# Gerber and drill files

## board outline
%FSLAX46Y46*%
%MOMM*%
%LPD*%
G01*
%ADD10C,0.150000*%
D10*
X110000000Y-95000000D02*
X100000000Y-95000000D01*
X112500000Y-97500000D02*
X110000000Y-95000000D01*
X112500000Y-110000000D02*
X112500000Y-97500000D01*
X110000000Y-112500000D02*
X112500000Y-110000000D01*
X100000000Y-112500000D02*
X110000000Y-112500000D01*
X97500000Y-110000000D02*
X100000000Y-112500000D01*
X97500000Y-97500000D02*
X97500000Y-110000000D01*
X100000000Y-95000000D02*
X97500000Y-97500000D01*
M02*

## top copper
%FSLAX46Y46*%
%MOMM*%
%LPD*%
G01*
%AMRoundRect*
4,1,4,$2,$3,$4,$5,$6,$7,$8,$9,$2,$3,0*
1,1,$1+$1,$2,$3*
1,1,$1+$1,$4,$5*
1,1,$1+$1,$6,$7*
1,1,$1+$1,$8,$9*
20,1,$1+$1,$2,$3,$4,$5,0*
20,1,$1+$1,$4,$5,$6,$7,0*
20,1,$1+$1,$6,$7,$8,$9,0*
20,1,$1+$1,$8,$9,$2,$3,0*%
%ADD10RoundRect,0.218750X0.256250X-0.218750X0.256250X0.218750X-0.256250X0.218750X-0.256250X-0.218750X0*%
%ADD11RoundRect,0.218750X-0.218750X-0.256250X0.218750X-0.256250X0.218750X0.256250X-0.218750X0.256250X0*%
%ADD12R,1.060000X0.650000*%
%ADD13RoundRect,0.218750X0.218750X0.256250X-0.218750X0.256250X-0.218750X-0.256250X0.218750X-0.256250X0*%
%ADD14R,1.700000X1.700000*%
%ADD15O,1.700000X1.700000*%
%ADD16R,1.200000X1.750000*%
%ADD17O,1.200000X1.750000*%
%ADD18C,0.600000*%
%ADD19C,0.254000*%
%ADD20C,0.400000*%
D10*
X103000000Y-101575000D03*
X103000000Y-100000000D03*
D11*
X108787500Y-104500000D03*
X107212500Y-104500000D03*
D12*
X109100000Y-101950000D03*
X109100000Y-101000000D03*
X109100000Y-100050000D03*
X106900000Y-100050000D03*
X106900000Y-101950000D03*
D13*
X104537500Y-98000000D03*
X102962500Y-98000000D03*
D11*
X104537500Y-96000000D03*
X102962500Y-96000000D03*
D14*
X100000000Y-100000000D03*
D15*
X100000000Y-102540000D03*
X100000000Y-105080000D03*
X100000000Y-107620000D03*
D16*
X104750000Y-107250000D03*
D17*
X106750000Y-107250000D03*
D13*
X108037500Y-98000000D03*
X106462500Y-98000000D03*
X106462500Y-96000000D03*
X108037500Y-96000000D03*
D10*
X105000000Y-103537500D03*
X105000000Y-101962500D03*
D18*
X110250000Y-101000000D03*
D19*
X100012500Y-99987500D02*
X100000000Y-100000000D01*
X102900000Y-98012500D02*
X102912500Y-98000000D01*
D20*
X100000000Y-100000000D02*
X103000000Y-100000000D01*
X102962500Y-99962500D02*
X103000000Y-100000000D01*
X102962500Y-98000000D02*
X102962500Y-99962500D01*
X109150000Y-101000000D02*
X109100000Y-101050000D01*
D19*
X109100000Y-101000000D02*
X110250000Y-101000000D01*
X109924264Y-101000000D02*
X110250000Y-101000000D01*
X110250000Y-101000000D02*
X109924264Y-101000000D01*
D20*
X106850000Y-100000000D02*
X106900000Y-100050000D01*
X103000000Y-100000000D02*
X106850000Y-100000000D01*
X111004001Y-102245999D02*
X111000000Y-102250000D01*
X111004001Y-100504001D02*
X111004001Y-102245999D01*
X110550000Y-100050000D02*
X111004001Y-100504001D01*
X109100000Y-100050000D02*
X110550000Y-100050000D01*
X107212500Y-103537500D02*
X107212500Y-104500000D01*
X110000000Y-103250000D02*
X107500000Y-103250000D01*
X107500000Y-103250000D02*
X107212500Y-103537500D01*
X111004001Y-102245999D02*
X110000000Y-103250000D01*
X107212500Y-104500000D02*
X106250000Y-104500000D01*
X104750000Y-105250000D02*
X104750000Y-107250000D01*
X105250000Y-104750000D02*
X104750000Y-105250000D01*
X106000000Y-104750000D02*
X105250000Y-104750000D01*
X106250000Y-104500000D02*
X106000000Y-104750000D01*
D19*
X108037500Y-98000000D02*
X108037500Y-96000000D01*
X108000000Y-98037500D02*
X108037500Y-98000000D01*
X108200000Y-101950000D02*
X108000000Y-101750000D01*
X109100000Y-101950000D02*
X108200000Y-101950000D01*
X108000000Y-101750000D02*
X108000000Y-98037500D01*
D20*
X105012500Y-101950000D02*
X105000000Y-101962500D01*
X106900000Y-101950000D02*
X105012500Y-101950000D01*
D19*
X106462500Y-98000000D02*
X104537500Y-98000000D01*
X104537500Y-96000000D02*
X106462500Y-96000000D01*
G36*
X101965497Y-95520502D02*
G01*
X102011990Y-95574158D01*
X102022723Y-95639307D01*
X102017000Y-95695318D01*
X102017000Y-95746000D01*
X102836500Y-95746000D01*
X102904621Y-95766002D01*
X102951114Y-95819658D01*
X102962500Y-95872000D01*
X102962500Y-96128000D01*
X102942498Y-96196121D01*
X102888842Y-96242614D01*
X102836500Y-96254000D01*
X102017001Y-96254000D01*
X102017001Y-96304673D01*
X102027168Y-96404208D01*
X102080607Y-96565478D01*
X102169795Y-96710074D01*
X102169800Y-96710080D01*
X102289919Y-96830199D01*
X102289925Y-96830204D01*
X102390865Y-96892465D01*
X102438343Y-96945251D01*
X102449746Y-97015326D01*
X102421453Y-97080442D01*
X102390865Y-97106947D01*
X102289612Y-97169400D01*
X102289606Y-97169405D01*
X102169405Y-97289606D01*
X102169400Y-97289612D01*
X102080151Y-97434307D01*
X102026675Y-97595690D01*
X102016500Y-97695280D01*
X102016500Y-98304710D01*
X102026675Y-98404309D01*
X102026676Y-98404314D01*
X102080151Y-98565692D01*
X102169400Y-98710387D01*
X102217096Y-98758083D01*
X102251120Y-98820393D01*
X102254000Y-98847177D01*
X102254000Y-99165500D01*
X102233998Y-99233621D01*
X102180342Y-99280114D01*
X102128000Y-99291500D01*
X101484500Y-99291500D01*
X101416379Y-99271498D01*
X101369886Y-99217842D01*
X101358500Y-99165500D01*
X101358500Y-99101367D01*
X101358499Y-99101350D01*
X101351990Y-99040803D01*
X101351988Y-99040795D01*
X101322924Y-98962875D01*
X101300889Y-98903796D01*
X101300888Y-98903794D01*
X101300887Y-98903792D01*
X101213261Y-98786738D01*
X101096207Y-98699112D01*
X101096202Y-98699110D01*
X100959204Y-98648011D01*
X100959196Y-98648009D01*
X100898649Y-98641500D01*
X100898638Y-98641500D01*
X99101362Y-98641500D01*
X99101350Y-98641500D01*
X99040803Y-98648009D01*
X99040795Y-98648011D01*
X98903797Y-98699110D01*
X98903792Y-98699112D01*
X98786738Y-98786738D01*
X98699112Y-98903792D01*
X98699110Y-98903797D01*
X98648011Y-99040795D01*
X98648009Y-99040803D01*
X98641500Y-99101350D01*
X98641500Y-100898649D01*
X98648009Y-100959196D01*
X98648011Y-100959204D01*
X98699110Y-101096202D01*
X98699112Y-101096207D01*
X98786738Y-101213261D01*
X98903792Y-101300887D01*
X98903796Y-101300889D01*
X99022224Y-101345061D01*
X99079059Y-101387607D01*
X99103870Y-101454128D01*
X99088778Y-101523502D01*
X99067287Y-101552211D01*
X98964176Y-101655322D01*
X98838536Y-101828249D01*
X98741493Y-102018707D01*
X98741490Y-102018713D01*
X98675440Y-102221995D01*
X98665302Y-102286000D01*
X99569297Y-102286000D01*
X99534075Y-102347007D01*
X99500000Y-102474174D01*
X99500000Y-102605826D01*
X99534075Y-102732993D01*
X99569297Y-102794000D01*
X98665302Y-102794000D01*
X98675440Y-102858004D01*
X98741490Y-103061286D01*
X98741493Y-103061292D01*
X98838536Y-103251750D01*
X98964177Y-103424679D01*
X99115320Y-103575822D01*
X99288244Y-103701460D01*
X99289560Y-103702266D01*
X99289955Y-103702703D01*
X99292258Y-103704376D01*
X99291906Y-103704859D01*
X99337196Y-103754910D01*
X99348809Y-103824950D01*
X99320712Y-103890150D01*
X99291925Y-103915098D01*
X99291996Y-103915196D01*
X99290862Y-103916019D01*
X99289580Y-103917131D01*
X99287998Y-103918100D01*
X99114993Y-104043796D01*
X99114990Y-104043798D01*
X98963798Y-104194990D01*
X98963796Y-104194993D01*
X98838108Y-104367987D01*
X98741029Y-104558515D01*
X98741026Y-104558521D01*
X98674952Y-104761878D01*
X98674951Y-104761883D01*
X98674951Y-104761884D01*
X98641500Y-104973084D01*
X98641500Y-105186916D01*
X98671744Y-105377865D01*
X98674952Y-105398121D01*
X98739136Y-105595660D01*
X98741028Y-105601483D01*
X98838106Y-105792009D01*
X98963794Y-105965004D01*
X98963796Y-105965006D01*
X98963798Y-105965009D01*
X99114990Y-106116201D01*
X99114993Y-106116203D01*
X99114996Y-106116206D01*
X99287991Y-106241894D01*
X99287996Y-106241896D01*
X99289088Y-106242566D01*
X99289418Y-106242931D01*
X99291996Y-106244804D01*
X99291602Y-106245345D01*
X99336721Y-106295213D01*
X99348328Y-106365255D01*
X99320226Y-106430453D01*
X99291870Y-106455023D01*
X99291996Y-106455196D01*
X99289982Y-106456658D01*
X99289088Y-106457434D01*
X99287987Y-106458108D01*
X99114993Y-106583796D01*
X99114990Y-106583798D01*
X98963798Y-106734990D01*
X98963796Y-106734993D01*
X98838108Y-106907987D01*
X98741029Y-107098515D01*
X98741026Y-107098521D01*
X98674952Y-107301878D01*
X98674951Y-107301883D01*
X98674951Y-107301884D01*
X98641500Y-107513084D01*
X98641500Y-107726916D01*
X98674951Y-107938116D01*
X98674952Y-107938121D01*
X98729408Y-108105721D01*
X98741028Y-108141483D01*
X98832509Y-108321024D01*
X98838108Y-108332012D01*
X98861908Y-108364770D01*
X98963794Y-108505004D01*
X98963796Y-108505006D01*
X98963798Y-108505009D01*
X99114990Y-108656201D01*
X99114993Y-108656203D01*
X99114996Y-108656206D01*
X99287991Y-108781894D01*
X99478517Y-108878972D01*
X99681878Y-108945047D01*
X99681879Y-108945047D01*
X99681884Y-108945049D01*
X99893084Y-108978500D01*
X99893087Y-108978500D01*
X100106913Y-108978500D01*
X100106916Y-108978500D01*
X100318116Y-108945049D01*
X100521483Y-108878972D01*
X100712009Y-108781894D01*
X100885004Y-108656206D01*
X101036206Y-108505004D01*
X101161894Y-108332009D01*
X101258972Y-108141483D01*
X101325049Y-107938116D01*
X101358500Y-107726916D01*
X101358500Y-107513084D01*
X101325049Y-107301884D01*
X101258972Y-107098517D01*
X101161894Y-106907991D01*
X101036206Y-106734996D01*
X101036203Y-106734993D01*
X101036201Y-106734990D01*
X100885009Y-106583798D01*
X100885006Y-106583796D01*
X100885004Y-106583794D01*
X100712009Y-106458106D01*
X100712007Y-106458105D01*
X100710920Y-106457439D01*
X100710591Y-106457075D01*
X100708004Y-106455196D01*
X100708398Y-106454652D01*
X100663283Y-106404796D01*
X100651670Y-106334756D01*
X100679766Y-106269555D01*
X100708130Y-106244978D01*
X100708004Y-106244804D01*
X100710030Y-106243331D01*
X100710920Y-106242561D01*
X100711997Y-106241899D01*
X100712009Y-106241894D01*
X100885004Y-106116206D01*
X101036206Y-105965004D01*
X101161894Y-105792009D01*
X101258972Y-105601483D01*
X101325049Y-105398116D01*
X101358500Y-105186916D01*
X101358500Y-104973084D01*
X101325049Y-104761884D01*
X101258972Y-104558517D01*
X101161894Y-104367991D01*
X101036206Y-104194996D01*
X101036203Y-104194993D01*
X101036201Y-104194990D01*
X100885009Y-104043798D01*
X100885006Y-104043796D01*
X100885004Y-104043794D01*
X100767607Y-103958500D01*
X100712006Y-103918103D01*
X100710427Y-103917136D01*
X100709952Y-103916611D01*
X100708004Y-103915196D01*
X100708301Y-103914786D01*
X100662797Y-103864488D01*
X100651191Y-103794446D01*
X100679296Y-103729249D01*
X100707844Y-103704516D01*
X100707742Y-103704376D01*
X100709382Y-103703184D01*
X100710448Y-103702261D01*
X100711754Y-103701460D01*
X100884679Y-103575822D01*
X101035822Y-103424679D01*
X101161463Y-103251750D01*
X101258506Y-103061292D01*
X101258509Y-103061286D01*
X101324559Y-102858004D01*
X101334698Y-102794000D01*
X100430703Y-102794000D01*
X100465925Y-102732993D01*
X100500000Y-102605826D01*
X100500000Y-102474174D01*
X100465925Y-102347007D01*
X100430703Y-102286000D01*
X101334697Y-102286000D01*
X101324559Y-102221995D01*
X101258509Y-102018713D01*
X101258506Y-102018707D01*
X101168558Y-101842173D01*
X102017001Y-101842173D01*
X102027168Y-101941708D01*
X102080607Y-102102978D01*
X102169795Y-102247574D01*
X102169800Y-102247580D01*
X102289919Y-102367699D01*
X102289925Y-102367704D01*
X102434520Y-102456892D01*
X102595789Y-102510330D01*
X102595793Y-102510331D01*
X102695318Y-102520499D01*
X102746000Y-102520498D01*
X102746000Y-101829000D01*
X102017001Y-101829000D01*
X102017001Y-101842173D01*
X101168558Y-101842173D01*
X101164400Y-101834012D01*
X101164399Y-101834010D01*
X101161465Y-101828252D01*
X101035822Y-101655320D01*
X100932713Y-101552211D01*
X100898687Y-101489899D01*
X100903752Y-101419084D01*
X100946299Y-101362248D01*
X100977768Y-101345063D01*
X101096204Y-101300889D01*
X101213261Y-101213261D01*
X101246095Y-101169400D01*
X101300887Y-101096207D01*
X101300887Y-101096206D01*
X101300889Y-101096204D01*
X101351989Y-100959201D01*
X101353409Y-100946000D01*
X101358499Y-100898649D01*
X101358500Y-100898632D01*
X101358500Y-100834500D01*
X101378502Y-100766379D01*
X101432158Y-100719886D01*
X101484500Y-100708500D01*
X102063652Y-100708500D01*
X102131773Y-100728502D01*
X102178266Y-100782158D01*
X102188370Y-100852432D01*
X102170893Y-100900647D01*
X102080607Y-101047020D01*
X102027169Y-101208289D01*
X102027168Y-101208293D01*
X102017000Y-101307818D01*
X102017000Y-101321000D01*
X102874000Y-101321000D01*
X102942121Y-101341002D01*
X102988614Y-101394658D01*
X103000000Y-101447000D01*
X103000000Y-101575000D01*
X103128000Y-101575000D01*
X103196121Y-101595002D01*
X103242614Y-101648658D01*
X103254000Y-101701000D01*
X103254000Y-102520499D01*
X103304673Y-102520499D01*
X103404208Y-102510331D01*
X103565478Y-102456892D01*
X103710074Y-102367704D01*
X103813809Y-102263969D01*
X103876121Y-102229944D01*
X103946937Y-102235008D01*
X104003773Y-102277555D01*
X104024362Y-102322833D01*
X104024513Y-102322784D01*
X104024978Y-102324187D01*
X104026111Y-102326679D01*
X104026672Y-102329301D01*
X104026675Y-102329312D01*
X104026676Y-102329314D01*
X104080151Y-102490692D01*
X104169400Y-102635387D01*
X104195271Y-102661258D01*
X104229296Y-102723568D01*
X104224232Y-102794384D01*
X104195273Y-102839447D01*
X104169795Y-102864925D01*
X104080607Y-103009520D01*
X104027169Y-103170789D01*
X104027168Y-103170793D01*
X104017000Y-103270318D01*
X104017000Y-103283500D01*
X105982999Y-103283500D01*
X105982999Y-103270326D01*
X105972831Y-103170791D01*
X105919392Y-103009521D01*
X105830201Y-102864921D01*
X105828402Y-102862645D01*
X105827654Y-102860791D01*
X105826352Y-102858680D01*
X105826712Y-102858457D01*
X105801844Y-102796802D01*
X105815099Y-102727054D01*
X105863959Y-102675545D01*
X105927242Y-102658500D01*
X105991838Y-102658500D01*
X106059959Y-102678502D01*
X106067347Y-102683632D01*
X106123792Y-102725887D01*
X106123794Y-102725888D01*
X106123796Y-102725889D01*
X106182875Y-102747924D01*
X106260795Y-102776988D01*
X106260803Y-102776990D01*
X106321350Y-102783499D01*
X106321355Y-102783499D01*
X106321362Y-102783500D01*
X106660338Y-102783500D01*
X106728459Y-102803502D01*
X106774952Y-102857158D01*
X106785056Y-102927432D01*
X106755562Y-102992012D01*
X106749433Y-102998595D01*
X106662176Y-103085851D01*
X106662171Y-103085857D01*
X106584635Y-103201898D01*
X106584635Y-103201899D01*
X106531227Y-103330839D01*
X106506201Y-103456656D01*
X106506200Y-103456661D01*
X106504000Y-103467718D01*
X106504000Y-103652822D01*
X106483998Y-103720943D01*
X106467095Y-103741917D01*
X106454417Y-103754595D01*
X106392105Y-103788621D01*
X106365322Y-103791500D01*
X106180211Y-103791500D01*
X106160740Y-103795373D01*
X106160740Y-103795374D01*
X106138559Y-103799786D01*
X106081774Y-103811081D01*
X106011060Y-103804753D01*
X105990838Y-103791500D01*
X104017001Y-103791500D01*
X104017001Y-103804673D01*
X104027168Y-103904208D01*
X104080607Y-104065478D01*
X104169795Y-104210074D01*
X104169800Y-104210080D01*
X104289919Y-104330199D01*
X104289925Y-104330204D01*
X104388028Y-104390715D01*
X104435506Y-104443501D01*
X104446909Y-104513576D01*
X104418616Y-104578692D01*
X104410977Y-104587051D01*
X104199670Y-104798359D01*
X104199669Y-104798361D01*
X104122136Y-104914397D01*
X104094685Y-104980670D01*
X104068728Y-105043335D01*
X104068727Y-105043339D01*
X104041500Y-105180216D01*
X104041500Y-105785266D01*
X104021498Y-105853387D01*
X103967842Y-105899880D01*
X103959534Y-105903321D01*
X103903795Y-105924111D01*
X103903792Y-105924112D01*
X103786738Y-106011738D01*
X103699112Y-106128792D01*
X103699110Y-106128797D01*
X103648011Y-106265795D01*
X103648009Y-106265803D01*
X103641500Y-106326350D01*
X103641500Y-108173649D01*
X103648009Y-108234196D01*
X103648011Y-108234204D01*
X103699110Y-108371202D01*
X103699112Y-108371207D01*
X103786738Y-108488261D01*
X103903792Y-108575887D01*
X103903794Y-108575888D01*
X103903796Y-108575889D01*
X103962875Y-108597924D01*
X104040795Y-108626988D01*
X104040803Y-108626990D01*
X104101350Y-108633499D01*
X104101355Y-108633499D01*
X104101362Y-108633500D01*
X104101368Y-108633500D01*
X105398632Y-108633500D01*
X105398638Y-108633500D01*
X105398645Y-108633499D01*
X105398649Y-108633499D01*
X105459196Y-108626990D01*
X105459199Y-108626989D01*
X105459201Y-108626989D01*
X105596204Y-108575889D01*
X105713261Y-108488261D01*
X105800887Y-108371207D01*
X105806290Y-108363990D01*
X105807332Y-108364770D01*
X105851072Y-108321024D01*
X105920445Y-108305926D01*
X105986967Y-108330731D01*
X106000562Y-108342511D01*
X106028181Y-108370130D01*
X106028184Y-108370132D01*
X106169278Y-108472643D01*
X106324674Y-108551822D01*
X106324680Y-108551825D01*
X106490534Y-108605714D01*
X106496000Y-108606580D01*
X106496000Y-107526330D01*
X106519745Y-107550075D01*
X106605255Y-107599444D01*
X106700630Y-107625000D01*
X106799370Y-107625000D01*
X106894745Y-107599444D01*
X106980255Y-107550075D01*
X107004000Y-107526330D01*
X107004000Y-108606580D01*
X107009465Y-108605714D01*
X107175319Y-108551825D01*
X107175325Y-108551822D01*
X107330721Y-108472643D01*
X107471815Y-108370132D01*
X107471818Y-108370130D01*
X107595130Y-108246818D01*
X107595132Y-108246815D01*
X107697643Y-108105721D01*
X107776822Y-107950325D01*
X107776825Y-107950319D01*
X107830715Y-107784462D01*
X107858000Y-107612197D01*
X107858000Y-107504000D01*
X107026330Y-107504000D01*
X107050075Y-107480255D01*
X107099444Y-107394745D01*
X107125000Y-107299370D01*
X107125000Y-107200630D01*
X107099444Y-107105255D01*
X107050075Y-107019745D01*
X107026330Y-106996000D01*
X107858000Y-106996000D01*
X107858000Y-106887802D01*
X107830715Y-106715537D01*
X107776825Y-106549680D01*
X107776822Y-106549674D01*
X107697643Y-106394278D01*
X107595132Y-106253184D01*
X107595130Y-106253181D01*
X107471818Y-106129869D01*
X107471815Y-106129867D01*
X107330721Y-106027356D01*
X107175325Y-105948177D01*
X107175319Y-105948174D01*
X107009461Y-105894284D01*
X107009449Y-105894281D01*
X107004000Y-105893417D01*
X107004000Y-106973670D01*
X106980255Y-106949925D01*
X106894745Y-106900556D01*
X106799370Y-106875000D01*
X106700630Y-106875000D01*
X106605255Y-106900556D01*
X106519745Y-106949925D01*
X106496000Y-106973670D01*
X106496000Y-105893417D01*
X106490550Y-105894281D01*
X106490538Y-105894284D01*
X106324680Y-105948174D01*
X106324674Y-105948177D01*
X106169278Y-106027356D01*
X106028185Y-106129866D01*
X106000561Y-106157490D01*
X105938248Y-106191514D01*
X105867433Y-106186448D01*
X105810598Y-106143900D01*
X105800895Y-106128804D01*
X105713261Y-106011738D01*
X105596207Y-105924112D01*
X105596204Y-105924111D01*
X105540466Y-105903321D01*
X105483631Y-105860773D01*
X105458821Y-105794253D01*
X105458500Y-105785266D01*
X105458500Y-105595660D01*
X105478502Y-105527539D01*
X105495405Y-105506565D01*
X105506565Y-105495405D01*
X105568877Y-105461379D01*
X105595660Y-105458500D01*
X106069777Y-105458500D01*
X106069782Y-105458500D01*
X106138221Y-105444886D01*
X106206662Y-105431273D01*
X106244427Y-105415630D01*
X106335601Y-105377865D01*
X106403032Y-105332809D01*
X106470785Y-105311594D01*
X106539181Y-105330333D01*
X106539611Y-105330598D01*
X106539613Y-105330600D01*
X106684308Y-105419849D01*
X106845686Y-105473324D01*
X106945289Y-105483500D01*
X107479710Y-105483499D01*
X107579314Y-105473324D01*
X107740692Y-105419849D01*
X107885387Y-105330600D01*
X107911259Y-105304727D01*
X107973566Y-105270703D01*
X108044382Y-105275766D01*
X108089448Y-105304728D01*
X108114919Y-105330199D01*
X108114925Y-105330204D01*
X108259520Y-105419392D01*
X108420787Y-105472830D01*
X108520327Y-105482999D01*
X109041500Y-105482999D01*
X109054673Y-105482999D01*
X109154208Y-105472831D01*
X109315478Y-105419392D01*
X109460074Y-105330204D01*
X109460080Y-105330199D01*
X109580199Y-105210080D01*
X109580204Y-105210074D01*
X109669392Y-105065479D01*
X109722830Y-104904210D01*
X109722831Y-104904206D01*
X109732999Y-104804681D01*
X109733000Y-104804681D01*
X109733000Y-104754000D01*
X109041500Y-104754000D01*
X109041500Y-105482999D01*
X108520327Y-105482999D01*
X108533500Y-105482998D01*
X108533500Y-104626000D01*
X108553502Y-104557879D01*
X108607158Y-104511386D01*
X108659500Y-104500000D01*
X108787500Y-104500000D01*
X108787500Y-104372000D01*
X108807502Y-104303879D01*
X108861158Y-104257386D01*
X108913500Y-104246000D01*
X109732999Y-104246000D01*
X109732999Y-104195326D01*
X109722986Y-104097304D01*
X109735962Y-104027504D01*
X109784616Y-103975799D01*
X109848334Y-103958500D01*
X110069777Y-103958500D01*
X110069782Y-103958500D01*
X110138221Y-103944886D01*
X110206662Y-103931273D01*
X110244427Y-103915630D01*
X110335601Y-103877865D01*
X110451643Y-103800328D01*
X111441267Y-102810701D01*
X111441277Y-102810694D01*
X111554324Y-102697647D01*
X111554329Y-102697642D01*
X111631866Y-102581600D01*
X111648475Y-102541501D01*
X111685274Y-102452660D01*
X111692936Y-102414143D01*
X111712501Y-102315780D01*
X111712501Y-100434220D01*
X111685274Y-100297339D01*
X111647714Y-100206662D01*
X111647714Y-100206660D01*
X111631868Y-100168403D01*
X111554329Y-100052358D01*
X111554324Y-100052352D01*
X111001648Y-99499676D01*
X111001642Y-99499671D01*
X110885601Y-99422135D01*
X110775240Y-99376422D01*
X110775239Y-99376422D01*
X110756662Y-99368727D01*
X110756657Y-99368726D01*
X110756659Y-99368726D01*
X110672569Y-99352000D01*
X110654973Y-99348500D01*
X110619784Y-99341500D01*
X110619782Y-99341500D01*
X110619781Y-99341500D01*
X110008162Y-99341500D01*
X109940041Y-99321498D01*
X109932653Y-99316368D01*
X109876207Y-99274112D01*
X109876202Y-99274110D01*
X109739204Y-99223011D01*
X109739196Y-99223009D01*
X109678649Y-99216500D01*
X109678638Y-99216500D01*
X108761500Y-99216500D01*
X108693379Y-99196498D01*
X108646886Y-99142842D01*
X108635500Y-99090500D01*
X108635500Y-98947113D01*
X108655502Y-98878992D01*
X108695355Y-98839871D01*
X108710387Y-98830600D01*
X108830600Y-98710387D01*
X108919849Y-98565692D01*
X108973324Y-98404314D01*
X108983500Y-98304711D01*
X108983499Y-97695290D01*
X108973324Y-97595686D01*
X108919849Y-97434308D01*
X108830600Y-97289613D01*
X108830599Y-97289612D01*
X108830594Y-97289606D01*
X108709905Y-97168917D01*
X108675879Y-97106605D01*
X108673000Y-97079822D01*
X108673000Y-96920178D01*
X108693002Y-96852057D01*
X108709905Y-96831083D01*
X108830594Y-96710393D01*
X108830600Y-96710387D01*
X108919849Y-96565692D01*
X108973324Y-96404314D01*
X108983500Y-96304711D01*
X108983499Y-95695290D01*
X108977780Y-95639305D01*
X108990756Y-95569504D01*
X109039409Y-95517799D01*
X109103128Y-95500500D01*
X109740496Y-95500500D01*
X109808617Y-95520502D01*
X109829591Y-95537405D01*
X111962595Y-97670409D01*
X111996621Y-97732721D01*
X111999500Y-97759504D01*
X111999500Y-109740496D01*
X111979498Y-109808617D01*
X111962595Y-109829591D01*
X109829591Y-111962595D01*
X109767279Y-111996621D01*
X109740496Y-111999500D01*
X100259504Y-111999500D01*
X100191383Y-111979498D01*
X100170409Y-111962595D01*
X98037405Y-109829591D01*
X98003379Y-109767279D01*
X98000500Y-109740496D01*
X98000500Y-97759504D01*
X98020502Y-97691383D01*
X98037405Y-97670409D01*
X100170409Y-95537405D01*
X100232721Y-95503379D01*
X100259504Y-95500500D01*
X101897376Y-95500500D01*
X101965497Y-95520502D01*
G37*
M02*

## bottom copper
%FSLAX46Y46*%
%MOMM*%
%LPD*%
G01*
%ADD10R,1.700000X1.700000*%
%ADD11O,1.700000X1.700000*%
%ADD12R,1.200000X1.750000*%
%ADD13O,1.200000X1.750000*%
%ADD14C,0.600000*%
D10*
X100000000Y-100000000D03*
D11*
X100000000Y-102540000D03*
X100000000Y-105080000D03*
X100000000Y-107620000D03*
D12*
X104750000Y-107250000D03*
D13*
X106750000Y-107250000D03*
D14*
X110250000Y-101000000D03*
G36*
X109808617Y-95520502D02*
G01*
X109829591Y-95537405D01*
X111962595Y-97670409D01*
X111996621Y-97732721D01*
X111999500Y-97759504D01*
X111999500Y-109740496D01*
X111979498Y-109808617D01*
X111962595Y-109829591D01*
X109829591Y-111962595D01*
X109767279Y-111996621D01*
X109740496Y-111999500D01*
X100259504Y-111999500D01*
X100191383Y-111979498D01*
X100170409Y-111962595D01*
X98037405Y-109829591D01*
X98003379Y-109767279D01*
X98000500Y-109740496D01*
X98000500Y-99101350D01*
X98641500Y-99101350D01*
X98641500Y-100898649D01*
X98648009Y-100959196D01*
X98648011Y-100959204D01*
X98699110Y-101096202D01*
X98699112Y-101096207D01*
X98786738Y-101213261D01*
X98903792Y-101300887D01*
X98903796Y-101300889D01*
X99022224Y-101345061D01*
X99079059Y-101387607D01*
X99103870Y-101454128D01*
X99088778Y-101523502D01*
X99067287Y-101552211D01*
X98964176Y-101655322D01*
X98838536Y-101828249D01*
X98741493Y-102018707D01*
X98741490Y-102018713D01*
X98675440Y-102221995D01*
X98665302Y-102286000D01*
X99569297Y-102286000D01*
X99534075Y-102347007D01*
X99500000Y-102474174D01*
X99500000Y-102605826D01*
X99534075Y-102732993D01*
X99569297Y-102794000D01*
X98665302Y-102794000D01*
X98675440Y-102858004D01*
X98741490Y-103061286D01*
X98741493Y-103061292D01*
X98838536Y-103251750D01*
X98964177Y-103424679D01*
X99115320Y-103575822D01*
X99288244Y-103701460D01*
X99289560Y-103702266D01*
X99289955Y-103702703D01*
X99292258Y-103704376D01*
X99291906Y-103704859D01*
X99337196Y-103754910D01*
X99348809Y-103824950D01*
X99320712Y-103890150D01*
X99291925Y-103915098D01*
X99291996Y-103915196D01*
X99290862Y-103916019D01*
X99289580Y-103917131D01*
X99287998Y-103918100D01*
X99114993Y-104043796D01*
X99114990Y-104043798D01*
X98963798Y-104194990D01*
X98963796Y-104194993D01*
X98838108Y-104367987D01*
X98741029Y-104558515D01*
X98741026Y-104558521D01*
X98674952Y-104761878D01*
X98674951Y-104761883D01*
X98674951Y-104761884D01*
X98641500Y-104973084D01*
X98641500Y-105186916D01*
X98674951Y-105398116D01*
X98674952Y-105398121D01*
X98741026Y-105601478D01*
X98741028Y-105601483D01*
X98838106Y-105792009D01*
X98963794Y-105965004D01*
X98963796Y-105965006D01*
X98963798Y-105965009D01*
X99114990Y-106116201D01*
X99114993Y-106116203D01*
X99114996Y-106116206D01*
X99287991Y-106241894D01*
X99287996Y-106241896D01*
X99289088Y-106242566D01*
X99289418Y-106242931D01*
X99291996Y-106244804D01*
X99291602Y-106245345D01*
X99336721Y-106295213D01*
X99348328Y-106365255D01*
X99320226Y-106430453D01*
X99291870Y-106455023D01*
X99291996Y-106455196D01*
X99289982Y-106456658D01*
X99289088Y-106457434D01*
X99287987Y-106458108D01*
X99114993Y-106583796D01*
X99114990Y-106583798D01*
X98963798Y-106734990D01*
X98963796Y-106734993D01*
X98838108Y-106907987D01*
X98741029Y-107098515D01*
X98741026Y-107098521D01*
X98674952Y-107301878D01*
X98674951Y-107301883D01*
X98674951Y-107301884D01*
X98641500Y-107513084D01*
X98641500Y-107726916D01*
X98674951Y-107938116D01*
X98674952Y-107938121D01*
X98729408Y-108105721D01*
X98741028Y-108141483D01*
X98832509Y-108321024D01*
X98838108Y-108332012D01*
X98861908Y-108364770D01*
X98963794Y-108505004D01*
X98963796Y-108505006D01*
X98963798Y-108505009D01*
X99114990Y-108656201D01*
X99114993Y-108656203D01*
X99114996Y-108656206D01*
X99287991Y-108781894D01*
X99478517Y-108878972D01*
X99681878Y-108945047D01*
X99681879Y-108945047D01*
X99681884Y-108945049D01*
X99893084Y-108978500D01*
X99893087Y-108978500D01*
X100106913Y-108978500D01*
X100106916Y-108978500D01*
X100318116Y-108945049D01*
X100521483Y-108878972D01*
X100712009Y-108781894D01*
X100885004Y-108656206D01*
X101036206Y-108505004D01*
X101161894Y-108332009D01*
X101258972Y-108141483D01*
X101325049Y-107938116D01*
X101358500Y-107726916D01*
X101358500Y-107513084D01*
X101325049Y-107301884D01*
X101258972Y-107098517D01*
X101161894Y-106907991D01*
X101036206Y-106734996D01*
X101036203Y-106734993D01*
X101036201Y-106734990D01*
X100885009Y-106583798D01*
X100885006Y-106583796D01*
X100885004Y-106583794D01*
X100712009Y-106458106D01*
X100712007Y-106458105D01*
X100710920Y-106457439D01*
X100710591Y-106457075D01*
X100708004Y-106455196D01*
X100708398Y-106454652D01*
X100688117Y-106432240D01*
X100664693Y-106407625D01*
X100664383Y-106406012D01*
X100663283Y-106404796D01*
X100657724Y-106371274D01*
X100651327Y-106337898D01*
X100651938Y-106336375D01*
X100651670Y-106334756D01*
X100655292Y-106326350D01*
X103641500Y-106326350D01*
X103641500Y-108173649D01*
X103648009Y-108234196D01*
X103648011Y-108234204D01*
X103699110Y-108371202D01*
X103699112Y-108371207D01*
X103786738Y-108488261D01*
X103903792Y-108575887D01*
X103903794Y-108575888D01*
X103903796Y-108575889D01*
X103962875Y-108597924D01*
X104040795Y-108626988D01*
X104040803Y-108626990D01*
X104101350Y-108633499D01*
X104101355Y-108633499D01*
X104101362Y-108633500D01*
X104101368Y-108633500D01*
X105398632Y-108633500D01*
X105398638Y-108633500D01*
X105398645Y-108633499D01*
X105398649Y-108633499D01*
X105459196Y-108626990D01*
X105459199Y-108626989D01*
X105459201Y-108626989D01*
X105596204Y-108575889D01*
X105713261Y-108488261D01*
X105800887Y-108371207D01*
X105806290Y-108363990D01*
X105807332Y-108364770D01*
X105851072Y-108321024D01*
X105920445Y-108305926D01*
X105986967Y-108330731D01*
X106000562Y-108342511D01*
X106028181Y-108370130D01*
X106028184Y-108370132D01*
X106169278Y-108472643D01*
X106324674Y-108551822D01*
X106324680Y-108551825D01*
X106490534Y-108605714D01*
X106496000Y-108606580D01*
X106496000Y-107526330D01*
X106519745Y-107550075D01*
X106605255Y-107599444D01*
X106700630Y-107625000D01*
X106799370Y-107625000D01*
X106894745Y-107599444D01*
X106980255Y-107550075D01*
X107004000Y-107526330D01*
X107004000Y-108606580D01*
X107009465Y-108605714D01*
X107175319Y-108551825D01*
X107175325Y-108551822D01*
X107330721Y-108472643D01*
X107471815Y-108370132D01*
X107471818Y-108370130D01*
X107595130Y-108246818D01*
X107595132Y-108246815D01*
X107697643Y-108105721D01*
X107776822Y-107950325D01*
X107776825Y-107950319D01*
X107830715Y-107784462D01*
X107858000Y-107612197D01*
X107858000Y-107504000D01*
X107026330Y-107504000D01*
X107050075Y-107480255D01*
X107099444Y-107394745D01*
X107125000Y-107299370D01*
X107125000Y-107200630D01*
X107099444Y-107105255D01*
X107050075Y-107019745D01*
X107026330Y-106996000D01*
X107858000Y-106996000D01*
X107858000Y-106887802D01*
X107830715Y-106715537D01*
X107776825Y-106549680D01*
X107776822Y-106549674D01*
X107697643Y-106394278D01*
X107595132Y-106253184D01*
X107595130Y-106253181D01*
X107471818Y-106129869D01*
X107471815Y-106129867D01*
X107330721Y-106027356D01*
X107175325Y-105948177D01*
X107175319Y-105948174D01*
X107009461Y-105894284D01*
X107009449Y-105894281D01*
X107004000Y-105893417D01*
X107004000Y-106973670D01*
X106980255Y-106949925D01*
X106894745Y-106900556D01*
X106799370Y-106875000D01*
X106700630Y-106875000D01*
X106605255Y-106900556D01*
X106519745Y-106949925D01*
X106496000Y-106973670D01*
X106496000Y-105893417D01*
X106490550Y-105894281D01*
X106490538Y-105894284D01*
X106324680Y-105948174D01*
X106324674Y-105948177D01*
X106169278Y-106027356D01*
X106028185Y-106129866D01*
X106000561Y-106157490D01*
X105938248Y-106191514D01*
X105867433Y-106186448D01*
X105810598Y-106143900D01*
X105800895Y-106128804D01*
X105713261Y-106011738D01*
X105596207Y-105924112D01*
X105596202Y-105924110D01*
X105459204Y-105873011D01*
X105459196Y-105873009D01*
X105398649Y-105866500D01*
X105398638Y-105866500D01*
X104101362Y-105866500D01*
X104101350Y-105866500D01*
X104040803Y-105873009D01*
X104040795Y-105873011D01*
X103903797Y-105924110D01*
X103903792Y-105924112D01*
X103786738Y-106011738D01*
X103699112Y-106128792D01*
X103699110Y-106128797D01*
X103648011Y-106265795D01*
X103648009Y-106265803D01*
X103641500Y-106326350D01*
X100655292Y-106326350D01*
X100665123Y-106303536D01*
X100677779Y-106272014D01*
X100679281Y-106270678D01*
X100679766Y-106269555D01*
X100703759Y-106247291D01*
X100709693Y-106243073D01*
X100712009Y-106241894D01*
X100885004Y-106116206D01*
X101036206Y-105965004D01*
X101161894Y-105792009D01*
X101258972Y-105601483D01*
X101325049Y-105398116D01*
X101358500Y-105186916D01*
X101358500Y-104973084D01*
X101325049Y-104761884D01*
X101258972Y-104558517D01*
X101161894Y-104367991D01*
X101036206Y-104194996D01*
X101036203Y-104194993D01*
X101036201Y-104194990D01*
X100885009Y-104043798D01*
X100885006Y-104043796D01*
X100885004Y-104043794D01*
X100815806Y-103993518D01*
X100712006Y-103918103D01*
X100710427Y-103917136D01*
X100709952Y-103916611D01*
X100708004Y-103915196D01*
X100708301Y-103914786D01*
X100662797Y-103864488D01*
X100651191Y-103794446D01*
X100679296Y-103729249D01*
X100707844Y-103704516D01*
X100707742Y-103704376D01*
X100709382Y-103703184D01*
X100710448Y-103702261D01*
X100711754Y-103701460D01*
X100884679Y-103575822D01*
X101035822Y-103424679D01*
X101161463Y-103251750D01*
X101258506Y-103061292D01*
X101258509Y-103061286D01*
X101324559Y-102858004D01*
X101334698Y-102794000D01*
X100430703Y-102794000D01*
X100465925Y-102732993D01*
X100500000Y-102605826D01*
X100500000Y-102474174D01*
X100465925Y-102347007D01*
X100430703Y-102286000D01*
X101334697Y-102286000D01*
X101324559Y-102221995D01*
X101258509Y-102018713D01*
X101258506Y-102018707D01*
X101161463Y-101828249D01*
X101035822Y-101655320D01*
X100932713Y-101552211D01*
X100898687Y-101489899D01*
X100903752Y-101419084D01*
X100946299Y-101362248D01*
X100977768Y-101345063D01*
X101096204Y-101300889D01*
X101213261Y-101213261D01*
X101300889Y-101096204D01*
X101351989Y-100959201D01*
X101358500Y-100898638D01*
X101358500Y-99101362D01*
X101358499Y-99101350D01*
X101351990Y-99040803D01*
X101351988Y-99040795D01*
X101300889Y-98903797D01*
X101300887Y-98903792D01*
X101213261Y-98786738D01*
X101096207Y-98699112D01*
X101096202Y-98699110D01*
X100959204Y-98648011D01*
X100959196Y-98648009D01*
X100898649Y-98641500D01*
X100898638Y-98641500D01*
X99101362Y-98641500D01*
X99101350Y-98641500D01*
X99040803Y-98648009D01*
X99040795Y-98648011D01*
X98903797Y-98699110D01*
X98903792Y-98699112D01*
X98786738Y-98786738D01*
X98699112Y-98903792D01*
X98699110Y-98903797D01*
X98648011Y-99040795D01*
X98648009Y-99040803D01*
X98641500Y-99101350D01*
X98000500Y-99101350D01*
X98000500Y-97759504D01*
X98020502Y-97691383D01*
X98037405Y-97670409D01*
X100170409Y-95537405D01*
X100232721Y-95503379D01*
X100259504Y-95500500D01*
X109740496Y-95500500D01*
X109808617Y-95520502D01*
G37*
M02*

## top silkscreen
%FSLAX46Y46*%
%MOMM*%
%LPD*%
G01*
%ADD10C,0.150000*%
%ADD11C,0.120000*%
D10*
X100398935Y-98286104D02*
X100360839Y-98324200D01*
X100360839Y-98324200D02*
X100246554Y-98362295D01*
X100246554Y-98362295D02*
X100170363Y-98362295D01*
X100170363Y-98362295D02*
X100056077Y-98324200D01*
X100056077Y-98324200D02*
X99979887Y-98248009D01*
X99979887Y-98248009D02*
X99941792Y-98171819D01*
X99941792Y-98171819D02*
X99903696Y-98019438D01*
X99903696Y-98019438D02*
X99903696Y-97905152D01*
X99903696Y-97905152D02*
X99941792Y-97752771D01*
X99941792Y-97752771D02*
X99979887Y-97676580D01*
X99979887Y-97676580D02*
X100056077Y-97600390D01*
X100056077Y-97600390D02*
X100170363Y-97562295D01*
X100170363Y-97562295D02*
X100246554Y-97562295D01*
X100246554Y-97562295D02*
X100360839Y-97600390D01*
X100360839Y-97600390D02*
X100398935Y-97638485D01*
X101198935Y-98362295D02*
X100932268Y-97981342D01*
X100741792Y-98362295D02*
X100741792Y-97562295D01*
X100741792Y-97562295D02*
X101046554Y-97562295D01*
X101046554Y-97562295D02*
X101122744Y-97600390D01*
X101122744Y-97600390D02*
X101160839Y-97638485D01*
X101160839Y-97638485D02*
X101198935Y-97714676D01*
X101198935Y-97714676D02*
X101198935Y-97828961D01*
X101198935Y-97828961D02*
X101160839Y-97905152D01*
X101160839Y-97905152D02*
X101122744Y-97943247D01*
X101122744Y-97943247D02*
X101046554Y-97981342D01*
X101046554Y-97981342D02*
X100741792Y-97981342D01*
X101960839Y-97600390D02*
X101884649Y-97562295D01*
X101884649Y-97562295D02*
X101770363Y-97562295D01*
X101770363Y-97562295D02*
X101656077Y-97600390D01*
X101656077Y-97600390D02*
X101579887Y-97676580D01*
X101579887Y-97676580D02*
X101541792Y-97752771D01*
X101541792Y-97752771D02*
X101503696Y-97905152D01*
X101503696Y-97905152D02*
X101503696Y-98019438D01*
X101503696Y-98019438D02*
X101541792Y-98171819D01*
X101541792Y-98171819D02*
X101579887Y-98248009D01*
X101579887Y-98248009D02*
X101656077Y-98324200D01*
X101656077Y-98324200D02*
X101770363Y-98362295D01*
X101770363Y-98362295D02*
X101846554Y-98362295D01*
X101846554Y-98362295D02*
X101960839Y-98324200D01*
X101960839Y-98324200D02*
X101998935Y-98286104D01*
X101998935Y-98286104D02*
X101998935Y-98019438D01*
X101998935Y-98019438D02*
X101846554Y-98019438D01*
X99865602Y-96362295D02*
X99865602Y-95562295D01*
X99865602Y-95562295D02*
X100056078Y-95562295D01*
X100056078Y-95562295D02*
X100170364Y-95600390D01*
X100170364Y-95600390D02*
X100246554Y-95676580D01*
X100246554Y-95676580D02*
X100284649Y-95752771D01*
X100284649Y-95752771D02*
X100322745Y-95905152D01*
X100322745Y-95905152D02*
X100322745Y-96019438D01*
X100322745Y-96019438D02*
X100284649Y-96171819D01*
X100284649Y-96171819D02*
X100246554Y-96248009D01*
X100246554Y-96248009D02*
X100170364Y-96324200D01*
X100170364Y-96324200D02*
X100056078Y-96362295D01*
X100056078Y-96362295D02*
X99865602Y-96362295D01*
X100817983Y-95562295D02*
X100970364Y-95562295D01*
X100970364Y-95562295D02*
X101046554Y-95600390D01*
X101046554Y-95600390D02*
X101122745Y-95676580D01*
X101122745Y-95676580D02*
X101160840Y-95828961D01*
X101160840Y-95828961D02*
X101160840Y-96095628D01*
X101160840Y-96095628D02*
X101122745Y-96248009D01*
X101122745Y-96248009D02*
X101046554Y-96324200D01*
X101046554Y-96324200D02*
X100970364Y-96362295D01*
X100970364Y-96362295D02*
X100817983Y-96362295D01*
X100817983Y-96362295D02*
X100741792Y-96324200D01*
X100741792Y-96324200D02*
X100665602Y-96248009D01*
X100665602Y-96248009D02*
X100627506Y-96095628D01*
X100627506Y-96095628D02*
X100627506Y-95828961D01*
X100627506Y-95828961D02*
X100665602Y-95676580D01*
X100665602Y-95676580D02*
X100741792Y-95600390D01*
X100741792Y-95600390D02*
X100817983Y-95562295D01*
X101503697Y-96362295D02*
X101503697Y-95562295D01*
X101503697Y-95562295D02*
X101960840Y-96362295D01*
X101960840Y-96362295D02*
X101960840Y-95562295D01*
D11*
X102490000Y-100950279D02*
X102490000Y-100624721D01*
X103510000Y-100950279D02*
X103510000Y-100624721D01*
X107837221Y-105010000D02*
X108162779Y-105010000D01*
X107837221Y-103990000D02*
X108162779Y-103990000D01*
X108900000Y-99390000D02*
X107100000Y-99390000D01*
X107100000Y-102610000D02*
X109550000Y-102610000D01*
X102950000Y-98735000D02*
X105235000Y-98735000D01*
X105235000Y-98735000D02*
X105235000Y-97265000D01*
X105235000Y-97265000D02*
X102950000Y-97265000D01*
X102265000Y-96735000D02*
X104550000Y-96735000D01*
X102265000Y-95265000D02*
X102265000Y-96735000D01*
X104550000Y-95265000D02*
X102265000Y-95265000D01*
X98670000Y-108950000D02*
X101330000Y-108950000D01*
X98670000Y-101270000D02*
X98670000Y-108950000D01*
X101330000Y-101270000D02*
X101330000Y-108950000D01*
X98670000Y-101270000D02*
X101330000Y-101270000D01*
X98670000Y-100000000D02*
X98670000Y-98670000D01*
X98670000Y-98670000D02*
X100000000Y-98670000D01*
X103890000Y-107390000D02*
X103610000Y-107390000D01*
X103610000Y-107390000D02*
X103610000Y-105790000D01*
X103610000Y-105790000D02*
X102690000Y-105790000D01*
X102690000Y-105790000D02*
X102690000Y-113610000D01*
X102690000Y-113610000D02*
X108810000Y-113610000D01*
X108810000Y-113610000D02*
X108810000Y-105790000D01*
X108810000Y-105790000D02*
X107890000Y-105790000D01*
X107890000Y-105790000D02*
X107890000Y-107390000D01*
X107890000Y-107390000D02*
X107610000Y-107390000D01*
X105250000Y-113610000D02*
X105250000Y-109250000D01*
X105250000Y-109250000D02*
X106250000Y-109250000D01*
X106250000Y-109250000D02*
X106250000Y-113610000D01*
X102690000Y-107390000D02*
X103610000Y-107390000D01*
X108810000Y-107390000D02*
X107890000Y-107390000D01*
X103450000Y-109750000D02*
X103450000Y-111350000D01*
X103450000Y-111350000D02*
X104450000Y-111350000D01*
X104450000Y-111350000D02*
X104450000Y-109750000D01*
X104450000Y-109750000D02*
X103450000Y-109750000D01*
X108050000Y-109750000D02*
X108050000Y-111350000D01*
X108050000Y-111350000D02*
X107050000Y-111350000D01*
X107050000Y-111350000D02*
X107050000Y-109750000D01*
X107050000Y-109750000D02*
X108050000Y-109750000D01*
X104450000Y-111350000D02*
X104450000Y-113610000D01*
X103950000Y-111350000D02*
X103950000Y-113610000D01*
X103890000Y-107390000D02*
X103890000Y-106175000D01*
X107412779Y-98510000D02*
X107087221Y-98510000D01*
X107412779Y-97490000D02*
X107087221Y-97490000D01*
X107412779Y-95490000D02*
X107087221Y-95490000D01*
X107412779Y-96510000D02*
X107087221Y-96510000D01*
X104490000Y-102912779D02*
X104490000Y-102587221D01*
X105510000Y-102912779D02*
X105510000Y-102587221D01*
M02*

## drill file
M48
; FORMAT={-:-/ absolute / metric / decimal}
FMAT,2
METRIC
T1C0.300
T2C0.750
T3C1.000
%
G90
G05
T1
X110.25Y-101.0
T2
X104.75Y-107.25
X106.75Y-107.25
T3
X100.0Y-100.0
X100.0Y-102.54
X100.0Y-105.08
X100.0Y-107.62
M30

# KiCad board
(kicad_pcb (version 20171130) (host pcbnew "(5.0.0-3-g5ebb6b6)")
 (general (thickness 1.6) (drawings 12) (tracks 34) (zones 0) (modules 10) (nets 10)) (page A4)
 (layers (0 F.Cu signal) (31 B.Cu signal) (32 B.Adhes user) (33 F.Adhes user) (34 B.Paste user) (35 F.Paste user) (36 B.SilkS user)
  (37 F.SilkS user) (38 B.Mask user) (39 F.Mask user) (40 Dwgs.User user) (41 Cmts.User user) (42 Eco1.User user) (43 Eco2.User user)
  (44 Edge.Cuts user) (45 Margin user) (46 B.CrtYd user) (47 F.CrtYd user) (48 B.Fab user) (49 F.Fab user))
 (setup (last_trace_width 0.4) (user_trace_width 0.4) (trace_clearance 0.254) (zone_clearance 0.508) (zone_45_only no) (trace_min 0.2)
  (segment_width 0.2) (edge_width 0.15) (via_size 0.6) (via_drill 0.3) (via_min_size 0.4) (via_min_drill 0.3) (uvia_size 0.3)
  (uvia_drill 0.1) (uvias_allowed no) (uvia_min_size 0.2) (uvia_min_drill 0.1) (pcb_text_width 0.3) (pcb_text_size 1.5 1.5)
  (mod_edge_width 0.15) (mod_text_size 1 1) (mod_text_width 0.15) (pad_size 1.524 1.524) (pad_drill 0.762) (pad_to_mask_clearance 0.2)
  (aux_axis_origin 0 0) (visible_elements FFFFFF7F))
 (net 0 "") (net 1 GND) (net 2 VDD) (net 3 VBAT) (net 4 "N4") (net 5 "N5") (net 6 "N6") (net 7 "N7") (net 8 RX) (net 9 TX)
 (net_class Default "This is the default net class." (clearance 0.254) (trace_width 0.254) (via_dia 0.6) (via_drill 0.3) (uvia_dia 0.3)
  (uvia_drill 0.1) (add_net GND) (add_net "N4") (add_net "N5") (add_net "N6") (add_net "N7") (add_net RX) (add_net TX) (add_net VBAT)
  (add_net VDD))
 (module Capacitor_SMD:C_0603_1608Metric (layer F.Cu) (at 103 100.7875 90)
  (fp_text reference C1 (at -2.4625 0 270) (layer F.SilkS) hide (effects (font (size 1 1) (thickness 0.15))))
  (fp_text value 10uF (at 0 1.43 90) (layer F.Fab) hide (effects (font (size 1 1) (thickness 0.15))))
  (fp_line (start -0.162779 -0.51) (end 0.162779 -0.51) (layer F.SilkS) (width 0.12))
  (fp_line (start -0.162779 0.51) (end 0.162779 0.51) (layer F.SilkS) (width 0.12))
  (pad 1 smd roundrect (at -0.7875 0 90) (size 0.875 0.95) (layers F.Cu F.Paste F.Mask) (roundrect_rratio 0.25) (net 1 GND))
  (pad 2 smd roundrect (at 0.7875 0 90) (size 0.875 0.95) (layers F.Cu F.Paste F.Mask) (roundrect_rratio 0.25) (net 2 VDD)))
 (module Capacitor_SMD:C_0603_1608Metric (layer F.Cu) (at 108 104.5)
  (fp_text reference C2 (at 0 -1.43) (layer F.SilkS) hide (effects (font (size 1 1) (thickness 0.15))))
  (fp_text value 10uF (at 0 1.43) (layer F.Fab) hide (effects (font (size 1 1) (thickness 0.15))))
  (fp_line (start -0.162779 0.51) (end 0.162779 0.51) (layer F.SilkS) (width 0.12))
  (fp_line (start -0.162779 -0.51) (end 0.162779 -0.51) (layer F.SilkS) (width 0.12))
  (pad 2 smd roundrect (at 0.7875 0) (size 0.875 0.95) (layers F.Cu F.Paste F.Mask) (roundrect_rratio 0.25) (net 1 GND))
  (pad 1 smd roundrect (at -0.7875 0) (size 0.875 0.95) (layers F.Cu F.Paste F.Mask) (roundrect_rratio 0.25) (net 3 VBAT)))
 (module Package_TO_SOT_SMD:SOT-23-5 (layer F.Cu) (at 108 101 180)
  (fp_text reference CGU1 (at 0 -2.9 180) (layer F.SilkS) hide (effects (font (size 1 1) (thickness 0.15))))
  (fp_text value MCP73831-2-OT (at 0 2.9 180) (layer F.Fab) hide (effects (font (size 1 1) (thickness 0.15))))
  (fp_line (start -0.9 1.61) (end 0.9 1.61) (layer F.SilkS) (width 0.12))
  (fp_line (start 0.9 -1.61) (end -1.55 -1.61) (layer F.SilkS) (width 0.12))
  (pad 1 smd rect (at -1.1 -0.95 180) (size 1.06 0.65) (layers F.Cu F.Paste F.Mask) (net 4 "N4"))
  (pad 2 smd rect (at -1.1 0 180) (size 1.06 0.65) (layers F.Cu F.Paste F.Mask) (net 1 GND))
  (pad 3 smd rect (at -1.1 0.95 180) (size 1.06 0.65) (layers F.Cu F.Paste F.Mask) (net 3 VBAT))
  (pad 4 smd rect (at 1.1 0.95 180) (size 1.06 0.65) (layers F.Cu F.Paste F.Mask) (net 2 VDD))
  (pad 5 smd rect (at 1.1 -0.95 180) (size 1.06 0.65) (layers F.Cu F.Paste F.Mask) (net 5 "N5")))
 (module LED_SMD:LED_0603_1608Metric (layer F.Cu) (at 103.75 98 180)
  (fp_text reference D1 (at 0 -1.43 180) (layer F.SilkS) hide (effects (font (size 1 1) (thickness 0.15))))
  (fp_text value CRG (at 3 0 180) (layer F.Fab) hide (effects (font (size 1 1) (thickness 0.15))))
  (fp_line (start 0.8 -0.735) (end -1.485 -0.735) (layer F.SilkS) (width 0.12))
  (fp_line (start -1.485 -0.735) (end -1.485 0.735) (layer F.SilkS) (width 0.12))
  (fp_line (start -1.485 0.735) (end 0.8 0.735) (layer F.SilkS) (width 0.12))
  (pad 1 smd roundrect (at -0.7875 0 180) (size 0.875 0.95) (layers F.Cu F.Paste F.Mask) (roundrect_rratio 0.25) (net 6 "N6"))
  (pad 2 smd roundrect (at 0.7875 0 180) (size 0.875 0.95) (layers F.Cu F.Paste F.Mask) (roundrect_rratio 0.25) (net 2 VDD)))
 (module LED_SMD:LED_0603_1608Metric (layer F.Cu) (at 103.75 96)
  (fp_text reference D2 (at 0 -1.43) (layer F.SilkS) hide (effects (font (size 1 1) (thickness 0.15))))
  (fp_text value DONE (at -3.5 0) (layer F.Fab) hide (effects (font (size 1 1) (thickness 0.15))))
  (fp_line (start -1.485 0.735) (end 0.8 0.735) (layer F.SilkS) (width 0.12))
  (fp_line (start -1.485 -0.735) (end -1.485 0.735) (layer F.SilkS) (width 0.12))
  (fp_line (start 0.8 -0.735) (end -1.485 -0.735) (layer F.SilkS) (width 0.12))
  (pad 2 smd roundrect (at 0.7875 0) (size 0.875 0.95) (layers F.Cu F.Paste F.Mask) (roundrect_rratio 0.25) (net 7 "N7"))
  (pad 1 smd roundrect (at -0.7875 0) (size 0.875 0.95) (layers F.Cu F.Paste F.Mask) (roundrect_rratio 0.25) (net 1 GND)))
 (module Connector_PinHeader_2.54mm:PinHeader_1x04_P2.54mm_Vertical (layer F.Cu) (at 100 100)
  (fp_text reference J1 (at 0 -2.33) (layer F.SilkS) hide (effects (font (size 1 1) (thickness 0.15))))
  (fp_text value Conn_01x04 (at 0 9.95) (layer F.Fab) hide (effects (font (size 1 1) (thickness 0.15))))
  (fp_line (start -1.33 8.95) (end 1.33 8.95) (layer F.SilkS) (width 0.12))
  (fp_line (start -1.33 1.27) (end -1.33 8.95) (layer F.SilkS) (width 0.12))
  (fp_line (start 1.33 1.27) (end 1.33 8.95) (layer F.SilkS) (width 0.12))
  (fp_line (start -1.33 1.27) (end 1.33 1.27) (layer F.SilkS) (width 0.12))
  (fp_line (start -1.33 0) (end -1.33 -1.33) (layer F.SilkS) (width 0.12))
  (fp_line (start -1.33 -1.33) (end 0 -1.33) (layer F.SilkS) (width 0.12))
  (pad 1 thru_hole rect (at 0 0) (size 1.7 1.7) (drill 1) (layers *.Cu *.Mask) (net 2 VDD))
  (pad 2 thru_hole oval (at 0 2.54) (size 1.7 1.7) (drill 1) (layers *.Cu *.Mask) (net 1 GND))
  (pad 3 thru_hole oval (at 0 5.08) (size 1.7 1.7) (drill 1) (layers *.Cu *.Mask) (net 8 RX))
  (pad 4 thru_hole oval (at 0 7.62) (size 1.7 1.7) (drill 1) (layers *.Cu *.Mask) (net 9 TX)))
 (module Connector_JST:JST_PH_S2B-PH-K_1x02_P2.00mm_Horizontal (layer F.Cu) (at 104.75 107.25)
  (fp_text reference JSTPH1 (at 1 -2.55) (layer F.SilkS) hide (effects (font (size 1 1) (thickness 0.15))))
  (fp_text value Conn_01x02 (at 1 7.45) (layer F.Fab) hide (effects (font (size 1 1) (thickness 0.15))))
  (fp_line (start -0.86 0.14) (end -1.14 0.14) (layer F.SilkS) (width 0.12))
  (fp_line (start -1.14 0.14) (end -1.14 -1.46) (layer F.SilkS) (width 0.12))
  (fp_line (start -1.14 -1.46) (end -2.06 -1.46) (layer F.SilkS) (width 0.12))
  (fp_line (start -2.06 -1.46) (end -2.06 6.36) (layer F.SilkS) (width 0.12))
  (fp_line (start -2.06 6.36) (end 4.06 6.36) (layer F.SilkS) (width 0.12))
  (fp_line (start 4.06 6.36) (end 4.06 -1.46) (layer F.SilkS) (width 0.12))
  (fp_line (start 4.06 -1.46) (end 3.14 -1.46) (layer F.SilkS) (width 0.12))
  (fp_line (start 3.14 -1.46) (end 3.14 0.14) (layer F.SilkS) (width 0.12))
  (fp_line (start 3.14 0.14) (end 2.86 0.14) (layer F.SilkS) (width 0.12))
  (fp_line (start 0.5 6.36) (end 0.5 2) (layer F.SilkS) (width 0.12))
  (fp_line (start 0.5 2) (end 1.5 2) (layer F.SilkS) (width 0.12))
  (fp_line (start 1.5 2) (end 1.5 6.36) (layer F.SilkS) (width 0.12))
  (fp_line (start -2.06 0.14) (end -1.14 0.14) (layer F.SilkS) (width 0.12))
  (fp_line (start 4.06 0.14) (end 3.14 0.14) (layer F.SilkS) (width 0.12))
  (fp_line (start -1.3 2.5) (end -1.3 4.1) (layer F.SilkS) (width 0.12))
  (fp_line (start -1.3 4.1) (end -0.3 4.1) (layer F.SilkS) (width 0.12))
  (fp_line (start -0.3 4.1) (end -0.3 2.5) (layer F.SilkS) (width 0.12))
  (fp_line (start -0.3 2.5) (end -1.3 2.5) (layer F.SilkS) (width 0.12))
  (fp_line (start 3.3 2.5) (end 3.3 4.1) (layer F.SilkS) (width 0.12))
  (fp_line (start 3.3 4.1) (end 2.3 4.1) (layer F.SilkS) (width 0.12))
  (fp_line (start 2.3 4.1) (end 2.3 2.5) (layer F.SilkS) (width 0.12))
  (fp_line (start 2.3 2.5) (end 3.3 2.5) (layer F.SilkS) (width 0.12))
  (fp_line (start -0.3 4.1) (end -0.3 6.36) (layer F.SilkS) (width 0.12))
  (fp_line (start -0.8 4.1) (end -0.8 6.36) (layer F.SilkS) (width 0.12))
  (fp_line (start -0.86 0.14) (end -0.86 -1.075) (layer F.SilkS) (width 0.12))
  (pad 1 thru_hole rect (at 0 0) (size 1.2 1.75) (drill 0.75) (layers *.Cu *.Mask) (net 3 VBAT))
  (pad 2 thru_hole oval (at 2 0) (size 1.2 1.75) (drill 0.75) (layers *.Cu *.Mask) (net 1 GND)))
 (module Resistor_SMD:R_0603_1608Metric (layer F.Cu) (at 107.25 98 180)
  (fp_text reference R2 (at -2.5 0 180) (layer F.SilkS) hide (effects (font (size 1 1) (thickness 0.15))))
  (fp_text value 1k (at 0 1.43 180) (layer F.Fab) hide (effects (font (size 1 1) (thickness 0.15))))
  (fp_line (start -0.162779 -0.51) (end 0.162779 -0.51) (layer F.SilkS) (width 0.12))
  (fp_line (start -0.162779 0.51) (end 0.162779 0.51) (layer F.SilkS) (width 0.12))
  (pad 1 smd roundrect (at -0.7875 0 180) (size 0.875 0.95) (layers F.Cu F.Paste F.Mask) (roundrect_rratio 0.25) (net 4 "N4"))
  (pad 2 smd roundrect (at 0.7875 0 180) (size 0.875 0.95) (layers F.Cu F.Paste F.Mask) (roundrect_rratio 0.25) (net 6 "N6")))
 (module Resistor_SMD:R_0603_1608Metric (layer F.Cu) (at 107.25 96 180)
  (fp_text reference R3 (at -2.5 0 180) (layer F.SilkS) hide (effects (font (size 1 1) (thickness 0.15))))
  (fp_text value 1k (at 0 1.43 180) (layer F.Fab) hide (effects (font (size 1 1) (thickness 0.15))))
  (fp_line (start -0.162779 0.51) (end 0.162779 0.51) (layer F.SilkS) (width 0.12))
  (fp_line (start -0.162779 -0.51) (end 0.162779 -0.51) (layer F.SilkS) (width 0.12))
  (pad 2 smd roundrect (at 0.7875 0 180) (size 0.875 0.95) (layers F.Cu F.Paste F.Mask) (roundrect_rratio 0.25) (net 7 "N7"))
  (pad 1 smd roundrect (at -0.7875 0 180) (size 0.875 0.95) (layers F.Cu F.Paste F.Mask) (roundrect_rratio 0.25) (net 4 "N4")))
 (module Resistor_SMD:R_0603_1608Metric (layer F.Cu) (at 105 102.75 90)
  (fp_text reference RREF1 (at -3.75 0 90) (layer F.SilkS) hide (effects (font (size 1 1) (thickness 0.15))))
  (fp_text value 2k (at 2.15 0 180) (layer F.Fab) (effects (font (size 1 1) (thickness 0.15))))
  (fp_line (start -0.162779 -0.51) (end 0.162779 -0.51) (layer F.SilkS) (width 0.12))
  (fp_line (start -0.162779 0.51) (end 0.162779 0.51) (layer F.SilkS) (width 0.12))
  (pad 1 smd roundrect (at -0.7875 0 90) (size 0.875 0.95) (layers F.Cu F.Paste F.Mask) (roundrect_rratio 0.25) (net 1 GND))
  (pad 2 smd roundrect (at 0.7875 0 90) (size 0.875 0.95) (layers F.Cu F.Paste F.Mask) (roundrect_rratio 0.25) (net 5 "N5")))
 (gr_line (start 110 95) (end 100 95) (layer Edge.Cuts) (width 0.15))
 (gr_line (start 112.5 97.5) (end 110 95) (layer Edge.Cuts) (width 0.15))
 (gr_line (start 112.5 110) (end 112.5 97.5) (layer Edge.Cuts) (width 0.15))
 (gr_line (start 110 112.5) (end 112.5 110) (layer Edge.Cuts) (width 0.15))
 (gr_line (start 100 112.5) (end 110 112.5) (layer Edge.Cuts) (width 0.15))
 (gr_line (start 97.5 110) (end 100 112.5) (layer Edge.Cuts) (width 0.15))
 (gr_line (start 97.5 97.5) (end 97.5 110) (layer Edge.Cuts) (width 0.15))
 (gr_line (start 100 95) (end 97.5 97.5) (layer Edge.Cuts) (width 0.15))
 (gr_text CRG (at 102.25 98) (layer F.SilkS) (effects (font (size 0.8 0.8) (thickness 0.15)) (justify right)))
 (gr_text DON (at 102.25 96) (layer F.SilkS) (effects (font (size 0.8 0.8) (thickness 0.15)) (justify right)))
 (segment (start 100.0125 99.9875) (end 100 100) (width 0.254) (layer F.Cu) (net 2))
 (segment (start 102.9 98.0125) (end 102.9125 98) (width 0.254) (layer F.Cu) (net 2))
 (segment (start 100 100) (end 103 100) (width 0.4) (layer F.Cu) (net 2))
 (segment (start 102.9625 99.9625) (end 103 100) (width 0.4) (layer F.Cu) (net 2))
 (segment (start 102.9625 98) (end 102.9625 99.9625) (width 0.4) (layer F.Cu) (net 2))
 (segment (start 109.15 101) (end 109.1 101.05) (width 0.4) (layer F.Cu) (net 1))
 (segment (start 109.1 101) (end 110.25 101) (width 0.254) (layer F.Cu) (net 1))
 (segment (start 109.924264 101) (end 110.25 101) (width 0.254) (layer F.Cu) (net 1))
 (segment (start 110.25 101) (end 109.924264 101) (width 0.254) (layer F.Cu) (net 1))
 (via (at 110.25 101) (size 0.6) (drill 0.3) (layers F.Cu B.Cu) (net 1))
 (segment (start 106.85 100) (end 106.9 100.05) (width 0.4) (layer F.Cu) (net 2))
 (segment (start 103 100) (end 106.85 100) (width 0.4) (layer F.Cu) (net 2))
 (segment (start 111.004001 102.245999) (end 111 102.25) (width 0.4) (layer F.Cu) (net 3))
 (segment (start 111.004001 100.504001) (end 111.004001 102.245999) (width 0.4) (layer F.Cu) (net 3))
 (segment (start 110.55 100.05) (end 111.004001 100.504001) (width 0.4) (layer F.Cu) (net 3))
 (segment (start 109.1 100.05) (end 110.55 100.05) (width 0.4) (layer F.Cu) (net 3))
 (segment (start 107.2125 103.5375) (end 107.2125 104.5) (width 0.4) (layer F.Cu) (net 3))
 (segment (start 110 103.25) (end 107.5 103.25) (width 0.4) (layer F.Cu) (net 3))
 (segment (start 107.5 103.25) (end 107.2125 103.5375) (width 0.4) (layer F.Cu) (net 3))
 (segment (start 111.004001 102.245999) (end 110 103.25) (width 0.4) (layer F.Cu) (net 3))
 (segment (start 107.2125 104.5) (end 106.25 104.5) (width 0.4) (layer F.Cu) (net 3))
 (segment (start 104.75 105.25) (end 104.75 107.25) (width 0.4) (layer F.Cu) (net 3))
 (segment (start 105.25 104.75) (end 104.75 105.25) (width 0.4) (layer F.Cu) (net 3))
 (segment (start 106 104.75) (end 105.25 104.75) (width 0.4) (layer F.Cu) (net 3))
 (segment (start 106.25 104.5) (end 106 104.75) (width 0.4) (layer F.Cu) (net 3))
 (segment (start 108.0375 98) (end 108.0375 96) (width 0.254) (layer F.Cu) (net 4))
 (segment (start 108 98.0375) (end 108.0375 98) (width 0.254) (layer F.Cu) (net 4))
 (segment (start 108.2 101.95) (end 108 101.75) (width 0.254) (layer F.Cu) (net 4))
 (segment (start 109.1 101.95) (end 108.2 101.95) (width 0.254) (layer F.Cu) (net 4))
 (segment (start 108 101.75) (end 108 98.0375) (width 0.254) (layer F.Cu) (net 4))
 (segment (start 105.0125 101.95) (end 105 101.9625) (width 0.4) (layer F.Cu) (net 5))
 (segment (start 106.9 101.95) (end 105.0125 101.95) (width 0.4) (layer F.Cu) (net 5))
 (segment (start 106.4625 98) (end 104.5375 98) (width 0.254) (layer F.Cu) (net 6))
 (segment (start 104.5375 96) (end 106.4625 96) (width 0.254) (layer F.Cu) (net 7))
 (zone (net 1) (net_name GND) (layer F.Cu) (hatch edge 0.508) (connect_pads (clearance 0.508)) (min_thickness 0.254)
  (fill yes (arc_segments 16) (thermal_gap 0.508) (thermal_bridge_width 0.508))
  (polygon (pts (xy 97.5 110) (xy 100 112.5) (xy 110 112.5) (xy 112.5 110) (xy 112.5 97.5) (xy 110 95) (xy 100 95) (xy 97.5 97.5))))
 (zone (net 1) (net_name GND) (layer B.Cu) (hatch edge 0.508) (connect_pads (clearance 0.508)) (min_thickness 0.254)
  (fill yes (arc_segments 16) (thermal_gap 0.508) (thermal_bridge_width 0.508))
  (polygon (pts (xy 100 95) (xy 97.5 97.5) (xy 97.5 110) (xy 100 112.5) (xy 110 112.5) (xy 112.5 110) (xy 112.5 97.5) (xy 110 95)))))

